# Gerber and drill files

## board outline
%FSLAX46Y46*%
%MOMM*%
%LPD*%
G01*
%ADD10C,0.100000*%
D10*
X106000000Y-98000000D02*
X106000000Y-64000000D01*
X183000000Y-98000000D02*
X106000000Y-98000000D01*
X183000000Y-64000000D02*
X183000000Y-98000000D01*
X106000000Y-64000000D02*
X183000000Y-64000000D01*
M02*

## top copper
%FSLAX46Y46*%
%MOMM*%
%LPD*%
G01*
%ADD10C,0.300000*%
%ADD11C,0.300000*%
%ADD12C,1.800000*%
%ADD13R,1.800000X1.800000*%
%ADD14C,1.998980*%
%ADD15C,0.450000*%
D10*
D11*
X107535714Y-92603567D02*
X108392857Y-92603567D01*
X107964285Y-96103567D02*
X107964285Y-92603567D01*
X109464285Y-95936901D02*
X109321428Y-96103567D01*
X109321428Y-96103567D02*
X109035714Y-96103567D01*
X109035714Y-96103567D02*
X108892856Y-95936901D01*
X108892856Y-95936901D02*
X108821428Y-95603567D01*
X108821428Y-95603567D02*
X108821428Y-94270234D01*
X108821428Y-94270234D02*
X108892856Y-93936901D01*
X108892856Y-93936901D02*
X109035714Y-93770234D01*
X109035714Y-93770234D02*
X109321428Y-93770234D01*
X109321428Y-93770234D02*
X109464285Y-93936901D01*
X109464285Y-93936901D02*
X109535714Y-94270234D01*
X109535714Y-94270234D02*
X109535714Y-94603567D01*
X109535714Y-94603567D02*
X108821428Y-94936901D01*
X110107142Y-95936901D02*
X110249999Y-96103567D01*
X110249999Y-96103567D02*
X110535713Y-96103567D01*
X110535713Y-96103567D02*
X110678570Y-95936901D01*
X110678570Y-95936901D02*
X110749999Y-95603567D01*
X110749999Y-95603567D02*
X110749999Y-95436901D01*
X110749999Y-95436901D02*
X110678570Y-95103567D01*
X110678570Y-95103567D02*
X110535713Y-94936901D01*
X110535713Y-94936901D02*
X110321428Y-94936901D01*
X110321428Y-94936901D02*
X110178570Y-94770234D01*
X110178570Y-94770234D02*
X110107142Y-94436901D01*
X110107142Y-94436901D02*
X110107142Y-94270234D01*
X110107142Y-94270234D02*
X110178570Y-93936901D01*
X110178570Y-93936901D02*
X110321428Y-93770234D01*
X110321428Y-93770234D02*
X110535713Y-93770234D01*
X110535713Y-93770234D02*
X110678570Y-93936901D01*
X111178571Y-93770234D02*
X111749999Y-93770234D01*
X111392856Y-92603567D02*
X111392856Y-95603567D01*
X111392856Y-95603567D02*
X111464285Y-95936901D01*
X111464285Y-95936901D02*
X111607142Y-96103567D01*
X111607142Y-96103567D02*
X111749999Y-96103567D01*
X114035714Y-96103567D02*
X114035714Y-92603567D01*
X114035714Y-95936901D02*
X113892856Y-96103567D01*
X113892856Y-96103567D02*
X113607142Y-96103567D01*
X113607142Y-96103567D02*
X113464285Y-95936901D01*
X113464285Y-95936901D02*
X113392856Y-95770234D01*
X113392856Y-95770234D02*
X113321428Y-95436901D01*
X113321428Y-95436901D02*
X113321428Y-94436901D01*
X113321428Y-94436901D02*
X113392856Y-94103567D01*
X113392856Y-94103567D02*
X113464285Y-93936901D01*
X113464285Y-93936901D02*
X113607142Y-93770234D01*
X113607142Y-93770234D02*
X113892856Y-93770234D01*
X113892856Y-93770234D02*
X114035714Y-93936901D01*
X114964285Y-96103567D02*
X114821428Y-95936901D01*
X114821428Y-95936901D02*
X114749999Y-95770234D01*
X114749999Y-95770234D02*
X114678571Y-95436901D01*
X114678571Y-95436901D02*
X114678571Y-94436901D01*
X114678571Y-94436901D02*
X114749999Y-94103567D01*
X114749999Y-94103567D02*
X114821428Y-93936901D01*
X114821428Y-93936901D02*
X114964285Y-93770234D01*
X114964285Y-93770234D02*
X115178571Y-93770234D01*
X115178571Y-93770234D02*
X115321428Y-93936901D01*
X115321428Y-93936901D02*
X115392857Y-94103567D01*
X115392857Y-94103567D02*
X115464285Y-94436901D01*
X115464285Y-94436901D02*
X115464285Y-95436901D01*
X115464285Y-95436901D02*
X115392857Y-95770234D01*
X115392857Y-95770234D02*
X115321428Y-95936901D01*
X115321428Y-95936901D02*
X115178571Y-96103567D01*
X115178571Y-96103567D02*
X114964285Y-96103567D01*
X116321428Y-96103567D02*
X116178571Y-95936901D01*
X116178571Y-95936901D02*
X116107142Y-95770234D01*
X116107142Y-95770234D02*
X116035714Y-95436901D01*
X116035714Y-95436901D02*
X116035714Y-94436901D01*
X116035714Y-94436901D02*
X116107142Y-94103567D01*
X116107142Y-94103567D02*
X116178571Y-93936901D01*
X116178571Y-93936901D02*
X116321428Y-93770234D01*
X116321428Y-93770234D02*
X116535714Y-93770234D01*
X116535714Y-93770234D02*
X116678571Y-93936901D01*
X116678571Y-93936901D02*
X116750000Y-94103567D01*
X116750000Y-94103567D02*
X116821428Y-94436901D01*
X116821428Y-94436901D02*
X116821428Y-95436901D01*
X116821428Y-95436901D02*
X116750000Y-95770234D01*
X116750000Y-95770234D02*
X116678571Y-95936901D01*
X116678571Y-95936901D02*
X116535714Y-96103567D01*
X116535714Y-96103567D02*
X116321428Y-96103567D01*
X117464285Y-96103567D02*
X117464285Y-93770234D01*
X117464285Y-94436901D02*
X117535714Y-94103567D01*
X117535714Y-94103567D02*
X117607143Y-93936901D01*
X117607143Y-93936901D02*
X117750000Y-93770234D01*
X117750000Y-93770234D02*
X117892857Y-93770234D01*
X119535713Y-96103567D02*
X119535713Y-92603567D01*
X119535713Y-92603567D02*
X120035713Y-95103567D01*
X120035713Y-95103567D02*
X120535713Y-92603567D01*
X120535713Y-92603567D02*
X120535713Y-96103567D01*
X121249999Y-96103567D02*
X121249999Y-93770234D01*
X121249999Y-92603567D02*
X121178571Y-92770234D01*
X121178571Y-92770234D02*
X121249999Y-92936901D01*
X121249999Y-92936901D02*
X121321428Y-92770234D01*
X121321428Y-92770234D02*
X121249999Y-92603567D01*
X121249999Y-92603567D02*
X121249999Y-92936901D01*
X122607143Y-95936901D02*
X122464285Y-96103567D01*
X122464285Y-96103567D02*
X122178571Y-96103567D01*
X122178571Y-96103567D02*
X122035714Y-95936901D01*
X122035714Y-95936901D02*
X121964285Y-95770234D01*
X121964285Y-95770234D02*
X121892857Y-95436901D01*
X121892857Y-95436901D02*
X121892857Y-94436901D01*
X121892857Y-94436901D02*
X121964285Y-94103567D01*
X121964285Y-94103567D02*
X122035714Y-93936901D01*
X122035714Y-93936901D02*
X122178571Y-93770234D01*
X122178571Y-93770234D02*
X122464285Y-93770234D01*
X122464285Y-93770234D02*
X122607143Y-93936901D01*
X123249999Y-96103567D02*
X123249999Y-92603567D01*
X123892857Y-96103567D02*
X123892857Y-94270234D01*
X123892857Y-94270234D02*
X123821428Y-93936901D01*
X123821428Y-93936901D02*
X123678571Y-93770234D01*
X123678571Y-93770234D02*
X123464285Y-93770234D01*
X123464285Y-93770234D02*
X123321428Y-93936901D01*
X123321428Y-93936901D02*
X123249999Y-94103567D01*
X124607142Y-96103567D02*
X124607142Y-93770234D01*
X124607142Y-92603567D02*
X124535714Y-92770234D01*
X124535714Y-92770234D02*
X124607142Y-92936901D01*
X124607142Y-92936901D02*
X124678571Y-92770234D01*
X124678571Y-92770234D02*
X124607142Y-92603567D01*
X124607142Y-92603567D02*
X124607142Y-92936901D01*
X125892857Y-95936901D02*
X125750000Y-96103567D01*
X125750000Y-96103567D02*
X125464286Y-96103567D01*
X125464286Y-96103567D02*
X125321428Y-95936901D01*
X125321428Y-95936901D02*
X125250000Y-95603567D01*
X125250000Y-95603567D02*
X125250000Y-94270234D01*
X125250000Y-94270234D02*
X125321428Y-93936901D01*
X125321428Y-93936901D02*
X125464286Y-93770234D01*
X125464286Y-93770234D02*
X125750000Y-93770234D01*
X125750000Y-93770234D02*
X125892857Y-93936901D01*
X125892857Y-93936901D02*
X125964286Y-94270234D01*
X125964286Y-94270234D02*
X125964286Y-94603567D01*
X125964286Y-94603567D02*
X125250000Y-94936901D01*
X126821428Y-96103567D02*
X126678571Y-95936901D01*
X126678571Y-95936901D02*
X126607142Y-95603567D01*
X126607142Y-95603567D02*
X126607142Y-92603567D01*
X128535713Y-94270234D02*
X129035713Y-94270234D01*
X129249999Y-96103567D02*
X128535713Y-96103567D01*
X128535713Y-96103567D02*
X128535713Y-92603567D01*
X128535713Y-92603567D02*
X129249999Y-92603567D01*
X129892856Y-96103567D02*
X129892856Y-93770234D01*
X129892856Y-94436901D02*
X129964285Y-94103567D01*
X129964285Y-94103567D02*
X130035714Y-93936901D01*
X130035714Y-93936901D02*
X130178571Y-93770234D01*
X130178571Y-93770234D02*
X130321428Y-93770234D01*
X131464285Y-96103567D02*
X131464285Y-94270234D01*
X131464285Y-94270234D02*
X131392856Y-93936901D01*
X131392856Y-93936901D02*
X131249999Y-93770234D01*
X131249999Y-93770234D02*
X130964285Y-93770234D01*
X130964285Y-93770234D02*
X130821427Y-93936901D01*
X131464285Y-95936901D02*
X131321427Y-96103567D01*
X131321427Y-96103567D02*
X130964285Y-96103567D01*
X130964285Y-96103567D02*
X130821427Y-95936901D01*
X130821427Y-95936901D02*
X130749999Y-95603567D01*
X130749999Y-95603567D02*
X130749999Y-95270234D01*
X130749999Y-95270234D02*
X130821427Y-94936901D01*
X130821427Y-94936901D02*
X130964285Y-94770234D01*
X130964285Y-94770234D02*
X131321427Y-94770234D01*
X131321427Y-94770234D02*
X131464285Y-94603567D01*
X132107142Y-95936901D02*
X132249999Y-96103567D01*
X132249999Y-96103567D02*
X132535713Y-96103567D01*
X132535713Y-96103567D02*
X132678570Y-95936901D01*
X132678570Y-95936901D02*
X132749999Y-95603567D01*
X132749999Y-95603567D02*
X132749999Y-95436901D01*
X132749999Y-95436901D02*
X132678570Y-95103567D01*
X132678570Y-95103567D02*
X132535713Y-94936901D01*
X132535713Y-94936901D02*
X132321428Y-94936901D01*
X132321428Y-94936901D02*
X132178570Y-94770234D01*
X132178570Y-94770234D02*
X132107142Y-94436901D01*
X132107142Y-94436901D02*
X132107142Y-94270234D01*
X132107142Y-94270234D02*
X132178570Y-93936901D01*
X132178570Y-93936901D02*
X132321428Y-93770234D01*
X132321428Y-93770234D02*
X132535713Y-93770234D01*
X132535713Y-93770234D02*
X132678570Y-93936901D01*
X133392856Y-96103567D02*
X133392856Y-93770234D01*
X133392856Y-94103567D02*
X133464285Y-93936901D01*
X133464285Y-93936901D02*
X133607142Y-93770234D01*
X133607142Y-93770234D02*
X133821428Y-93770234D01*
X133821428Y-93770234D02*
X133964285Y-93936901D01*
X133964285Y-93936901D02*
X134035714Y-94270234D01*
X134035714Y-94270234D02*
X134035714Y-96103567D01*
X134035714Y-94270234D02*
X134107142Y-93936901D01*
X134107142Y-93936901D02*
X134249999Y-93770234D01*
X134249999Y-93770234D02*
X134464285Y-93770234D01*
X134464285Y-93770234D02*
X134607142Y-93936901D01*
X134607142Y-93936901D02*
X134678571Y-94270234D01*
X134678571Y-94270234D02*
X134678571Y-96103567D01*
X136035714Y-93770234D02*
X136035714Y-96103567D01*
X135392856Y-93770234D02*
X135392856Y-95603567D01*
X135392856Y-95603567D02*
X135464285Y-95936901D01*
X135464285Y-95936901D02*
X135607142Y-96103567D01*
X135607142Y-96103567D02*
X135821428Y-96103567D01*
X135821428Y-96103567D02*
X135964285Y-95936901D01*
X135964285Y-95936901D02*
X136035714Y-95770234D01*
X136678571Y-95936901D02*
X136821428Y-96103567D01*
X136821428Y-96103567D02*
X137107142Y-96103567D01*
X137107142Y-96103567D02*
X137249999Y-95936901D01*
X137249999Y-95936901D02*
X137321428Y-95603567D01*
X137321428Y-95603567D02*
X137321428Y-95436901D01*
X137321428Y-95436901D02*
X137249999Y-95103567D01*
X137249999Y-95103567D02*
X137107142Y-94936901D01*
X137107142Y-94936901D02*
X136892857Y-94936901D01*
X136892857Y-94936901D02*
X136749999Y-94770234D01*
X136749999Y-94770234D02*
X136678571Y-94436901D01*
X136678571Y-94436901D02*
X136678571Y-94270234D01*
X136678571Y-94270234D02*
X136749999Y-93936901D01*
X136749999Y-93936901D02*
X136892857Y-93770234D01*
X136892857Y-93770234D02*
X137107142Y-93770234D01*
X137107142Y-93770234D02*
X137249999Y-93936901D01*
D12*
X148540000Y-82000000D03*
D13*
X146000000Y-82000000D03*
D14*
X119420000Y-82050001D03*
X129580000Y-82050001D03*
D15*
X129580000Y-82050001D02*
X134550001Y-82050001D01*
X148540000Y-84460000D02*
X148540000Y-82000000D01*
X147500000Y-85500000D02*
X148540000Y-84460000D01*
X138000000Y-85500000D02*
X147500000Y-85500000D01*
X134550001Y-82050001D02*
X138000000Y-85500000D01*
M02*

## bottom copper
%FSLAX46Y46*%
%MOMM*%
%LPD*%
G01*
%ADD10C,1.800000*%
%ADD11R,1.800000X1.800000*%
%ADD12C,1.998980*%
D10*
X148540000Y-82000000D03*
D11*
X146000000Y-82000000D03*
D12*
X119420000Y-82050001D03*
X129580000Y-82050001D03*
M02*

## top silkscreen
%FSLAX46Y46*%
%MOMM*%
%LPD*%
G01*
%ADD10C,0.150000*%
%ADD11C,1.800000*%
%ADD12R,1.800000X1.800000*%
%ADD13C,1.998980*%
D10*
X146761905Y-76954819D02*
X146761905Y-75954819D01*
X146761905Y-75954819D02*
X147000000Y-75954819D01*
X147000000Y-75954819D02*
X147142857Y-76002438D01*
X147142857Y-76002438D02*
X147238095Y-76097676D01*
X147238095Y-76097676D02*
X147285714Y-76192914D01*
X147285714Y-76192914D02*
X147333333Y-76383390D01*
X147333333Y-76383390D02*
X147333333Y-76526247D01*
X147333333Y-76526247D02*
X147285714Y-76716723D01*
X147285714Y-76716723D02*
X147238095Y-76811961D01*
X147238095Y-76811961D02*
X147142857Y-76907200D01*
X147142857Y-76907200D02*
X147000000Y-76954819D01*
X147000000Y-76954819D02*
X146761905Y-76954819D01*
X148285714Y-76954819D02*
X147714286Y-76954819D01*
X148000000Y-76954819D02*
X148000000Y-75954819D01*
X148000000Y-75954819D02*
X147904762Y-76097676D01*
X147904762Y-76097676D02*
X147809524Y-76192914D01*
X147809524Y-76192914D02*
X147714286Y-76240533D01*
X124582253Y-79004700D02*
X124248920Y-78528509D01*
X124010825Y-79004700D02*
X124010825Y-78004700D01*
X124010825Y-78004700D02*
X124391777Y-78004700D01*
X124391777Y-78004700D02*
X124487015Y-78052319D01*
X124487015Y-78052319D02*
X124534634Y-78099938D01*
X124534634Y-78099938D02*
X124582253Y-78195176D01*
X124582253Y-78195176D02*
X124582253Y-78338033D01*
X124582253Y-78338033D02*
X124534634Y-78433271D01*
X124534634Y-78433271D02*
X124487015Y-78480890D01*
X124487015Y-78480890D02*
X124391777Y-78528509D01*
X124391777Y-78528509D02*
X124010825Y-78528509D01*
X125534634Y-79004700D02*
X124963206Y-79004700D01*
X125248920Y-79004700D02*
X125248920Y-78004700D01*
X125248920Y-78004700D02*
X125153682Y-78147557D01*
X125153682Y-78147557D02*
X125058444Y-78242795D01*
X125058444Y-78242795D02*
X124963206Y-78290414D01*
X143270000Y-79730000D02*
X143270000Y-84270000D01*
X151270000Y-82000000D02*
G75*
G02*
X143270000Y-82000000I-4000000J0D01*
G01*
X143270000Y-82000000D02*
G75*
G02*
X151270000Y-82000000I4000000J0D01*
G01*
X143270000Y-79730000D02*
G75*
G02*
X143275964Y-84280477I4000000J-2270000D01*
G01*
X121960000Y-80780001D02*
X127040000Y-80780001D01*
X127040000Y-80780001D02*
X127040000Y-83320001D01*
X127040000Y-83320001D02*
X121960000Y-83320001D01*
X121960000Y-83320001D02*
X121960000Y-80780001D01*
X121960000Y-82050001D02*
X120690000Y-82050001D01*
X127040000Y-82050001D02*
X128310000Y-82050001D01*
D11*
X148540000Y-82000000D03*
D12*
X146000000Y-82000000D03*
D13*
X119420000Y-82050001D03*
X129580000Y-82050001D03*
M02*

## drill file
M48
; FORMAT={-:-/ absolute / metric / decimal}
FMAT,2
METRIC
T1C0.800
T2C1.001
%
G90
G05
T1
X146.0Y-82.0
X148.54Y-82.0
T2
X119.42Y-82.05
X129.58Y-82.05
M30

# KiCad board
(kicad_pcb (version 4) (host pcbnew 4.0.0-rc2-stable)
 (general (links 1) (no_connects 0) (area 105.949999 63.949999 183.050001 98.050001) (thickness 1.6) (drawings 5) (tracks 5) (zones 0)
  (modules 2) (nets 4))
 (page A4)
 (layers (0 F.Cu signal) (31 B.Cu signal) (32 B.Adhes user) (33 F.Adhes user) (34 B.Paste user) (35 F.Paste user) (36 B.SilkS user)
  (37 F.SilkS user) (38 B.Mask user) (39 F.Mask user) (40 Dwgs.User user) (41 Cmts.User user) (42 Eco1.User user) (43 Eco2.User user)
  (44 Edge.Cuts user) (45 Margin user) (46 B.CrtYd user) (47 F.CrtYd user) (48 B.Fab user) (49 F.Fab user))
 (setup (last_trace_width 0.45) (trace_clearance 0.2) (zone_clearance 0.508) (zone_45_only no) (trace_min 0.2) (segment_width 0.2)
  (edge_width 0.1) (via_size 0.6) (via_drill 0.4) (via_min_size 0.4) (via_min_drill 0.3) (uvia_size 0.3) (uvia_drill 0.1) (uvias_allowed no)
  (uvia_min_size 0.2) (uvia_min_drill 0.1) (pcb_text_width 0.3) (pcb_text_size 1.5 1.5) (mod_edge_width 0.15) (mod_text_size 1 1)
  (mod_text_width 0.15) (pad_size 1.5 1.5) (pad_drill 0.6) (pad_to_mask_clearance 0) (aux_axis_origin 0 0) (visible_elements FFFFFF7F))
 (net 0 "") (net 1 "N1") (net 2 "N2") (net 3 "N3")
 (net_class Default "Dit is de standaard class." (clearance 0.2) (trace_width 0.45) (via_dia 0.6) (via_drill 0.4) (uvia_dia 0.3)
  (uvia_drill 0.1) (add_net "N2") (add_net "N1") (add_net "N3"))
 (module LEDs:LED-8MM (layer F.Cu) (at 146 82)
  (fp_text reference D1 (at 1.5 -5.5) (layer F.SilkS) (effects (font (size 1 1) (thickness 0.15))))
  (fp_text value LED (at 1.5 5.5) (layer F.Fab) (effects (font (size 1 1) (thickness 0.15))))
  (fp_line (start -2.73 -2.27) (end -2.73 2.27) (layer F.SilkS) (width 0.15))
  (fp_circle (center 1.27 0) (end 1.27 4) (layer F.SilkS) (width 0.15))
  (fp_arc (start 1.27 0) (end -2.73 -2.27) (angle 300.7) (layer F.SilkS) (width 0.15))
  (pad 2 thru_hole circle (at 2.54 0 180) (size 1.8 1.8) (drill 0.8) (layers *.Cu *.Mask F.SilkS) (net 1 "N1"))
  (pad 1 thru_hole rect (at 0 0 180) (size 1.8 1.8) (drill 0.8) (layers *.Cu *.Mask F.SilkS) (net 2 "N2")))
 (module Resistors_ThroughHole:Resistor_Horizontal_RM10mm (layer F.Cu) (at 124.5 82.050001)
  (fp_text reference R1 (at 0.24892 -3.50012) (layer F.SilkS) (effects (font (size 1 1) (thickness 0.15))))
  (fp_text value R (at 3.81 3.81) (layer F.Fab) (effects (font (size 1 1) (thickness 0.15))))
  (fp_line (start -2.54 -1.27) (end 2.54 -1.27) (layer F.SilkS) (width 0.15))
  (fp_line (start 2.54 -1.27) (end 2.54 1.27) (layer F.SilkS) (width 0.15))
  (fp_line (start 2.54 1.27) (end -2.54 1.27) (layer F.SilkS) (width 0.15))
  (fp_line (start -2.54 1.27) (end -2.54 -1.27) (layer F.SilkS) (width 0.15))
  (fp_line (start -2.54 0) (end -3.81 0) (layer F.SilkS) (width 0.15))
  (fp_line (start 2.54 0) (end 3.81 0) (layer F.SilkS) (width 0.15))
  (pad 1 thru_hole circle (at -5.08 0) (size 1.99898 1.99898) (drill 1.00076) (layers *.Cu *.SilkS *.Mask) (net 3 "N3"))
  (pad 2 thru_hole circle (at 5.08 0) (size 1.99898 1.99898) (drill 1.00076) (layers *.Cu *.SilkS *.Mask) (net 1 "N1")))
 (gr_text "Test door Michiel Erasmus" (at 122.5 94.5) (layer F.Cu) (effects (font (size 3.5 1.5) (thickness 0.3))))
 (gr_line (start 106 98) (end 106 64) (angle 90) (layer Edge.Cuts) (width 0.1))
 (gr_line (start 183 98) (end 106 98) (angle 90) (layer Edge.Cuts) (width 0.1))
 (gr_line (start 183 64) (end 183 98) (angle 90) (layer Edge.Cuts) (width 0.1))
 (gr_line (start 106 64) (end 183 64) (angle 90) (layer Edge.Cuts) (width 0.1))
 (segment (start 129.58 82.050001) (end 134.550001 82.050001) (width 0.45) (layer F.Cu) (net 1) (status 400000))
 (segment (start 148.54 84.46) (end 148.54 82) (width 0.45) (layer F.Cu) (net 1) (status 800000))
 (segment (start 147.5 85.5) (end 148.54 84.46) (width 0.45) (layer F.Cu) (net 1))
 (segment (start 138 85.5) (end 147.5 85.5) (width 0.45) (layer F.Cu) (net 1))
 (segment (start 134.550001 82.050001) (end 138 85.5) (width 0.45) (layer F.Cu) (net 1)))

